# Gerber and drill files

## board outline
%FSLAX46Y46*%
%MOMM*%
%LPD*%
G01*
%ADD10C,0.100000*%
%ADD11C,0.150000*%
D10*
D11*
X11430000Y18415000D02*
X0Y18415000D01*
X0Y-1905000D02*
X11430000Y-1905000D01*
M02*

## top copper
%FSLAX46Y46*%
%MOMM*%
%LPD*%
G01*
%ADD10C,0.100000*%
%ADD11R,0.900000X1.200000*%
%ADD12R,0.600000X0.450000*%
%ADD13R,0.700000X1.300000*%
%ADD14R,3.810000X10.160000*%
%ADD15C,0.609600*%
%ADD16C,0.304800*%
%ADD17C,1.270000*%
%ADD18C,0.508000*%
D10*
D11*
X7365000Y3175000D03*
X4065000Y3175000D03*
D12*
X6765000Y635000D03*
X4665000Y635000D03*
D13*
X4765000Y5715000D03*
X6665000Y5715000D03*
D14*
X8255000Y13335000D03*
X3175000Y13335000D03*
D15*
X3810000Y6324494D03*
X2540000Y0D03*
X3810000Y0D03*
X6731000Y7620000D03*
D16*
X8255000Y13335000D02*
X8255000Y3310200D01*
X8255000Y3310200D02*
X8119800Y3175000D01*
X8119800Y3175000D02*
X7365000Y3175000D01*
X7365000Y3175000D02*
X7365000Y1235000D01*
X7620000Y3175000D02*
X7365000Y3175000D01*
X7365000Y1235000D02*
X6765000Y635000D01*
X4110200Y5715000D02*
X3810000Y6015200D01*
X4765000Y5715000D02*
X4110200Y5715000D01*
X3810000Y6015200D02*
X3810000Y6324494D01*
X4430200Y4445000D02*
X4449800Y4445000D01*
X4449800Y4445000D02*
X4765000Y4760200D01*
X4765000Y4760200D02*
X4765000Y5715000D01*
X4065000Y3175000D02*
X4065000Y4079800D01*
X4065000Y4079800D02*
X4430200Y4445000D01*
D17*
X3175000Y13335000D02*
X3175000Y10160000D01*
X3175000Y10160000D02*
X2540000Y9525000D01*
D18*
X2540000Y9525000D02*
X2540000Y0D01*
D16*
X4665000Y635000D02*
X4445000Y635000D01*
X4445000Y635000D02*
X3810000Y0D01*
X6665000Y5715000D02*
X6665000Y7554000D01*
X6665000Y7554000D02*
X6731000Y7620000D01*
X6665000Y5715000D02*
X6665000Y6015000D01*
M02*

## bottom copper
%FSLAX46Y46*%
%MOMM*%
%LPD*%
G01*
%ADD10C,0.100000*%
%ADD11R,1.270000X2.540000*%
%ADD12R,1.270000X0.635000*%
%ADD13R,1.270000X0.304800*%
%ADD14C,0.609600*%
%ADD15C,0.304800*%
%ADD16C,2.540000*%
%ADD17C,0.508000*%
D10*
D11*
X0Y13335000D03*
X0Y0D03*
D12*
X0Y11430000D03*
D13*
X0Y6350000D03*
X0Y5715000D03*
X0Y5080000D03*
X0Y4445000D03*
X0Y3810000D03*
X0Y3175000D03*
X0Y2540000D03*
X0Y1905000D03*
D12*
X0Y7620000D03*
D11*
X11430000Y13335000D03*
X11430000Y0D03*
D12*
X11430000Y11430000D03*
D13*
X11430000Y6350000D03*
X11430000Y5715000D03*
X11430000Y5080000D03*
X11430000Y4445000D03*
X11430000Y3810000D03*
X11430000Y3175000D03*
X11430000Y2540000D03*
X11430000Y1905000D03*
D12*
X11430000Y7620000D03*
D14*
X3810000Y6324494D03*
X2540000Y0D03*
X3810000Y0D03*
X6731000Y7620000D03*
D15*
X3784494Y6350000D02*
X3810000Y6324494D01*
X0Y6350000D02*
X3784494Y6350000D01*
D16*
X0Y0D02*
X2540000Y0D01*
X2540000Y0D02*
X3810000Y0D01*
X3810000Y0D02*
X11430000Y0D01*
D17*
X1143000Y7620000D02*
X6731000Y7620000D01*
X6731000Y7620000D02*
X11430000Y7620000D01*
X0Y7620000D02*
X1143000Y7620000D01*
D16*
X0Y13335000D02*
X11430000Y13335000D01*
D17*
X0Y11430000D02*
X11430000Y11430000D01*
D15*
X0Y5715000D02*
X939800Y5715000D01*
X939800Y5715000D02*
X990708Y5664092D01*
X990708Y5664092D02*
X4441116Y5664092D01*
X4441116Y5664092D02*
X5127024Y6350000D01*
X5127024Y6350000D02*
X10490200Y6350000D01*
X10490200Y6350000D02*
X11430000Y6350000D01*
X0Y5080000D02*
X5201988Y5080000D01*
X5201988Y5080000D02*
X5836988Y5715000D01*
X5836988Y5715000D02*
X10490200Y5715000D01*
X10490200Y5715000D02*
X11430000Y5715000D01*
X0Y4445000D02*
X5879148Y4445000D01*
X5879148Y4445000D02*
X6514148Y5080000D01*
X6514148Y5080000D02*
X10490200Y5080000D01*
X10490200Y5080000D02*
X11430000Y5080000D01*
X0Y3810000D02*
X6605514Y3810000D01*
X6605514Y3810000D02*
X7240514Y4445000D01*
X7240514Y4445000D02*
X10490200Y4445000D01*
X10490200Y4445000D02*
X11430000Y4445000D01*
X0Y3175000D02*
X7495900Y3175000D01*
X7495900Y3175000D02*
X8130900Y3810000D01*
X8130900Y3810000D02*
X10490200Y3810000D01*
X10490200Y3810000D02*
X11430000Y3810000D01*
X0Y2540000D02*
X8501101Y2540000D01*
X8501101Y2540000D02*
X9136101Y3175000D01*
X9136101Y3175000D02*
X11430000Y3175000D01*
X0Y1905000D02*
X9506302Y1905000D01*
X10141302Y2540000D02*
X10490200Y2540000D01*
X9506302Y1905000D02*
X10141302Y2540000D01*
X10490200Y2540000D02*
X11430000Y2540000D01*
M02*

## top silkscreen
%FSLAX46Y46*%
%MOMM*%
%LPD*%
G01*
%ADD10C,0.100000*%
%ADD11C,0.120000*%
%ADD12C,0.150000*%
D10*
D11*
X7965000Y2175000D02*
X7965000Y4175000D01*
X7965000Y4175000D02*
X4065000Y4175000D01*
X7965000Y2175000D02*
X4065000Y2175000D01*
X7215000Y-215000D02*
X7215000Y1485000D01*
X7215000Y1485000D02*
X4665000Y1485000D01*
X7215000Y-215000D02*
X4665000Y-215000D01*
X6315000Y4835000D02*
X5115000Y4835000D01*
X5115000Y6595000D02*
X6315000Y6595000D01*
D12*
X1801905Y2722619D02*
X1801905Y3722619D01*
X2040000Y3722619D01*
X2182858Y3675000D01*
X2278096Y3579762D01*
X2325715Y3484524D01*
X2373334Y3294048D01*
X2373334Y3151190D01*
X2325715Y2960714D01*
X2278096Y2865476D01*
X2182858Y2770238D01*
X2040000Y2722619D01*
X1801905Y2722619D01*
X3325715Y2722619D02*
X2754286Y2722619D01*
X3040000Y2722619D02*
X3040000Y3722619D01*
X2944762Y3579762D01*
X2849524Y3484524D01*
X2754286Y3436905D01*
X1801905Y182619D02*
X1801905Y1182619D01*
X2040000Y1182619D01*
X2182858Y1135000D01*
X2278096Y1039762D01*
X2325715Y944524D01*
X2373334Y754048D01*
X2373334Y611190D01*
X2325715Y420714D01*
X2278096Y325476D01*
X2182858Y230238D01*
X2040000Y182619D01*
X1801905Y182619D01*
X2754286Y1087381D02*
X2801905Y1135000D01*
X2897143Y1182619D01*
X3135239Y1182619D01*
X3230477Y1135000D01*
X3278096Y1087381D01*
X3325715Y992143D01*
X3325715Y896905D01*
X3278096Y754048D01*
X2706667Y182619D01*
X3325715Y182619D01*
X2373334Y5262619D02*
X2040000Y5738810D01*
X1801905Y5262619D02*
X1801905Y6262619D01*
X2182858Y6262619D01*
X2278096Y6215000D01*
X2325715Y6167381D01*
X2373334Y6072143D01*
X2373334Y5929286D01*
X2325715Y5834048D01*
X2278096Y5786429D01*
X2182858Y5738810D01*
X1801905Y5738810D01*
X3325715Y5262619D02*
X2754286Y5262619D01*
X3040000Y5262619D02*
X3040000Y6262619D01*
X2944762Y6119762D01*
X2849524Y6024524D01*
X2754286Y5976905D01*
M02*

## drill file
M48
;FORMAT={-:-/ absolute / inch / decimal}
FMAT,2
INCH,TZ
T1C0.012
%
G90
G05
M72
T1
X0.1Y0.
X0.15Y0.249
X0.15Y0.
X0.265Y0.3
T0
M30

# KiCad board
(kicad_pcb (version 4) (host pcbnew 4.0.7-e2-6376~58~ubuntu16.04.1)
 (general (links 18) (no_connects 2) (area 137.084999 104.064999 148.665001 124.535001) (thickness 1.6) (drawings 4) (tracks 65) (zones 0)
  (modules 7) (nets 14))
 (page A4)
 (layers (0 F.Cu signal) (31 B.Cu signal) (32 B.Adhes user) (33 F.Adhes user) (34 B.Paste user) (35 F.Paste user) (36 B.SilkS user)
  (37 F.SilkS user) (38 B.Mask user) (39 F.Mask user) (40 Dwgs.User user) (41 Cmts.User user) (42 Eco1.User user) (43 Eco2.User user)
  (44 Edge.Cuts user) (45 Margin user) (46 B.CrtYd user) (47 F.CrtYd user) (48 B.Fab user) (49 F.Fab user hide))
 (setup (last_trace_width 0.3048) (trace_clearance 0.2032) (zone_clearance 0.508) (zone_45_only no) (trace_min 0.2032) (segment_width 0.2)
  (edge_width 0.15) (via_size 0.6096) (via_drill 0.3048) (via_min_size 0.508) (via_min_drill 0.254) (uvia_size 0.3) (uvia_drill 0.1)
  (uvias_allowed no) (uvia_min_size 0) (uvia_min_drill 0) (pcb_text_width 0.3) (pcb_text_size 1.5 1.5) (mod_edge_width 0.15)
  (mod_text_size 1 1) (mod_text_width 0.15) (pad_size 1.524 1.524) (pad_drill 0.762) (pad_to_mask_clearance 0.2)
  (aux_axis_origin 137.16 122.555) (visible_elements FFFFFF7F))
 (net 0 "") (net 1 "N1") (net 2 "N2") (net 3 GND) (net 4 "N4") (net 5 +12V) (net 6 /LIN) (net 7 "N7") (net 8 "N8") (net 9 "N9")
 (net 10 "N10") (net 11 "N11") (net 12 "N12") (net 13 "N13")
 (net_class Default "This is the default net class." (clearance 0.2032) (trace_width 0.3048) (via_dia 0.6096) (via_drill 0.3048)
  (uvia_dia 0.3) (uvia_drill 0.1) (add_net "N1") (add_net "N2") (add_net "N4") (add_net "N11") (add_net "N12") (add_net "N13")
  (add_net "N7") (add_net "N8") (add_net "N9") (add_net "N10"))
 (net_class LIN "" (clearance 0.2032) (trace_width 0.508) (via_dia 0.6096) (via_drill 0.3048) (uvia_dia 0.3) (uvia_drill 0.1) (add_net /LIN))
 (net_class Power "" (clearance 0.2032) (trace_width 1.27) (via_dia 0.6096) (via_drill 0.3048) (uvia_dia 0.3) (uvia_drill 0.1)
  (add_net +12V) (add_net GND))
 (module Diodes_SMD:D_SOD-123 (layer F.Cu) (at 142.875 119.38 180)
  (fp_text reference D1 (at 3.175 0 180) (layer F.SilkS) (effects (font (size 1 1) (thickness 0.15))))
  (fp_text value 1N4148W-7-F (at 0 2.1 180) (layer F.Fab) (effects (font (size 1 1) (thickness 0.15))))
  (fp_line (start -2.25 -1) (end -2.25 1) (layer F.SilkS) (width 0.12))
  (fp_line (start -2.25 1) (end 1.65 1) (layer F.SilkS) (width 0.12))
  (fp_line (start -2.25 -1) (end 1.65 -1) (layer F.SilkS) (width 0.12))
  (pad 1 smd rect (at -1.65 0 180) (size 0.9 1.2) (layers F.Cu F.Paste F.Mask) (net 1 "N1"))
  (pad 2 smd rect (at 1.65 0 180) (size 0.9 1.2) (layers F.Cu F.Paste F.Mask) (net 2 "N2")))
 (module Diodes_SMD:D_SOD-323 (layer F.Cu) (at 142.875 121.92 180)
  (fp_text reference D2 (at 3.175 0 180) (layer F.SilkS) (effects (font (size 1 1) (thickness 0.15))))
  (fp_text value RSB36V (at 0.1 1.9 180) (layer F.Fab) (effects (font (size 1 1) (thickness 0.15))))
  (fp_line (start -1.5 -0.85) (end -1.5 0.85) (layer F.SilkS) (width 0.12))
  (fp_line (start -1.5 0.85) (end 1.05 0.85) (layer F.SilkS) (width 0.12))
  (fp_line (start -1.5 -0.85) (end 1.05 -0.85) (layer F.SilkS) (width 0.12))
  (pad 1 smd rect (at -1.05 0 180) (size 0.6 0.45) (layers F.Cu F.Paste F.Mask) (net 1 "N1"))
  (pad 2 smd rect (at 1.05 0 180) (size 0.6 0.45) (layers F.Cu F.Paste F.Mask) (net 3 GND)))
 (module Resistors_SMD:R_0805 (layer F.Cu) (at 142.875 116.84)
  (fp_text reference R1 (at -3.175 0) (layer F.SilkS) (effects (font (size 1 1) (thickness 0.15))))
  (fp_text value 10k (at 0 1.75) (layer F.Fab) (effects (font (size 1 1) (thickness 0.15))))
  (fp_line (start 0.6 0.88) (end -0.6 0.88) (layer F.SilkS) (width 0.12))
  (fp_line (start -0.6 -0.88) (end 0.6 -0.88) (layer F.SilkS) (width 0.12))
  (pad 1 smd rect (at -0.95 0) (size 0.7 1.3) (layers F.Cu F.Paste F.Mask) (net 2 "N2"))
  (pad 2 smd rect (at 0.95 0) (size 0.7 1.3) (layers F.Cu F.Paste F.Mask) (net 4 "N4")))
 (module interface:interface (layer F.Cu) (at 137.16 104.775)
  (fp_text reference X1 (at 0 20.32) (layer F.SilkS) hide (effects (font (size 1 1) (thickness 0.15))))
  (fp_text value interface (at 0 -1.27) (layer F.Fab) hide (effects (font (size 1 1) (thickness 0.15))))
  (pad 1 smd rect (at 0 4.445) (size 1.27 2.54) (layers B.Cu) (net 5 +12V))
  (pad 2 smd rect (at 0 17.78) (size 1.27 2.54) (layers B.Cu) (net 3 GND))
  (pad 3 smd rect (at 0 6.35) (size 1.27 0.635) (layers B.Cu) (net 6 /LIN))
  (pad 5 smd rect (at 0 11.43) (size 1.27 0.3048) (layers B.Cu) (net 2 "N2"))
  (pad 6 smd rect (at 0 12.065) (size 1.27 0.3048) (layers B.Cu) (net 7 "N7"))
  (pad 7 smd rect (at 0 12.7) (size 1.27 0.3048) (layers B.Cu) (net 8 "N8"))
  (pad 8 smd rect (at 0 13.335) (size 1.27 0.3048) (layers B.Cu) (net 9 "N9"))
  (pad 9 smd rect (at 0 13.97) (size 1.27 0.3048) (layers B.Cu) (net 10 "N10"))
  (pad 10 smd rect (at 0 14.605) (size 1.27 0.3048) (layers B.Cu) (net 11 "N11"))
  (pad 11 smd rect (at 0 15.24) (size 1.27 0.3048) (layers B.Cu) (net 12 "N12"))
  (pad 12 smd rect (at 0 15.875) (size 1.27 0.3048) (layers B.Cu) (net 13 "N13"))
  (pad 4 smd rect (at 0 10.16) (size 1.27 0.635) (layers B.Cu) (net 4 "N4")))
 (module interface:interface (layer F.Cu) (at 148.59 104.775)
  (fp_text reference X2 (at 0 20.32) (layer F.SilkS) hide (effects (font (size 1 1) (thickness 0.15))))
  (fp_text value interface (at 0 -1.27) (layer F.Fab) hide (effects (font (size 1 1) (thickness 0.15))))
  (pad 1 smd rect (at 0 4.445) (size 1.27 2.54) (layers B.Cu) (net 5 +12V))
  (pad 2 smd rect (at 0 17.78) (size 1.27 2.54) (layers B.Cu) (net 3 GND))
  (pad 3 smd rect (at 0 6.35) (size 1.27 0.635) (layers B.Cu) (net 6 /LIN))
  (pad 5 smd rect (at 0 11.43) (size 1.27 0.3048) (layers B.Cu) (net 7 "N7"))
  (pad 6 smd rect (at 0 12.065) (size 1.27 0.3048) (layers B.Cu) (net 8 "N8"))
  (pad 7 smd rect (at 0 12.7) (size 1.27 0.3048) (layers B.Cu) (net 9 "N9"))
  (pad 8 smd rect (at 0 13.335) (size 1.27 0.3048) (layers B.Cu) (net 10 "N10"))
  (pad 9 smd rect (at 0 13.97) (size 1.27 0.3048) (layers B.Cu) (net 11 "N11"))
  (pad 10 smd rect (at 0 14.605) (size 1.27 0.3048) (layers B.Cu) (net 12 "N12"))
  (pad 11 smd rect (at 0 15.24) (size 1.27 0.3048) (layers B.Cu) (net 13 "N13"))
  (pad 12 smd rect (at 0 15.875) (size 1.27 0.3048) (layers B.Cu))
  (pad 4 smd rect (at 0 10.16) (size 1.27 0.635) (layers B.Cu) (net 4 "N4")))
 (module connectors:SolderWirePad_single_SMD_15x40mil (layer F.Cu) (at 145.415 109.22)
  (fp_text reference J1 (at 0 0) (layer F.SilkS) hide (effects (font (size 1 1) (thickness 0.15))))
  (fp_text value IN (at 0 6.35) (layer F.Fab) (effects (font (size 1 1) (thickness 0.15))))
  (pad 1 smd rect (at 0 0) (size 3.81 10.16) (layers F.Cu F.Paste F.Mask) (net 1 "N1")))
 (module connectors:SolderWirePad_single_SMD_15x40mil (layer F.Cu) (at 140.335 109.22)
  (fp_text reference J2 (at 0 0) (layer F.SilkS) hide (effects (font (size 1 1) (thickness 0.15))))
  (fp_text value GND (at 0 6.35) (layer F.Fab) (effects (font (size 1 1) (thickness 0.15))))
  (pad 1 smd rect (at 0 0) (size 3.81 10.16) (layers F.Cu F.Paste F.Mask) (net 3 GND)))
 (gr_line (start 148.59 104.14) (end 137.16 104.14) (layer Edge.Cuts) (width 0.15))
 (gr_line (start 137.16 124.46) (end 148.59 124.46) (layer Edge.Cuts) (width 0.15))
 (segment (start 145.415 109.22) (end 145.415 119.2448) (width 0.3048) (layer F.Cu) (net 1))
 (segment (start 145.415 119.2448) (end 145.2798 119.38) (width 0.3048) (layer F.Cu) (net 1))
 (segment (start 145.2798 119.38) (end 144.525 119.38) (width 0.3048) (layer F.Cu) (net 1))
 (segment (start 144.525 119.38) (end 144.525 121.32) (width 0.3048) (layer F.Cu) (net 1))
 (segment (start 144.78 119.38) (end 144.525 119.38) (width 0.3048) (layer F.Cu) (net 1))
 (segment (start 144.525 121.32) (end 143.925 121.92) (width 0.3048) (layer F.Cu) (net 1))
 (segment (start 140.944494 116.205) (end 140.97 116.230506) (width 0.3048) (layer B.Cu) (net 2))
 (segment (start 137.16 116.205) (end 140.944494 116.205) (width 0.3048) (layer B.Cu) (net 2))
 (segment (start 141.2702 116.84) (end 140.97 116.5398) (width 0.3048) (layer F.Cu) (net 2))
 (segment (start 141.925 116.84) (end 141.2702 116.84) (width 0.3048) (layer F.Cu) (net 2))
 (segment (start 140.97 116.5398) (end 140.97 116.230506) (width 0.3048) (layer F.Cu) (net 2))
 (via (at 140.97 116.230506) (size 0.6096) (drill 0.3048) (layers F.Cu B.Cu) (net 2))
 (segment (start 141.5902 118.11) (end 141.6098 118.11) (width 0.3048) (layer F.Cu) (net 2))
 (segment (start 141.6098 118.11) (end 141.925 117.7948) (width 0.3048) (layer F.Cu) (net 2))
 (segment (start 141.925 117.7948) (end 141.925 116.84) (width 0.3048) (layer F.Cu) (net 2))
 (segment (start 141.225 119.38) (end 141.225 118.4752) (width 0.3048) (layer F.Cu) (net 2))
 (segment (start 141.225 118.4752) (end 141.5902 118.11) (width 0.3048) (layer F.Cu) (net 2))
 (segment (start 137.16 122.555) (end 139.7 122.555) (width 2.54) (layer B.Cu) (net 3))
 (segment (start 139.7 122.555) (end 140.97 122.555) (width 2.54) (layer B.Cu) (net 3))
 (segment (start 140.335 109.22) (end 140.335 112.395) (width 1.27) (layer F.Cu) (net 3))
 (segment (start 140.335 112.395) (end 139.7 113.03) (width 1.27) (layer F.Cu) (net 3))
 (segment (start 139.7 113.03) (end 139.7 122.555) (width 0.508) (layer F.Cu) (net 3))
 (via (at 139.7 122.555) (size 0.6096) (drill 0.3048) (layers F.Cu B.Cu) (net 3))
 (segment (start 140.97 122.555) (end 148.59 122.555) (width 2.54) (layer B.Cu) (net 3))
 (segment (start 141.825 121.92) (end 141.605 121.92) (width 0.3048) (layer F.Cu) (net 3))
 (segment (start 141.605 121.92) (end 140.97 122.555) (width 0.3048) (layer F.Cu) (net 3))
 (via (at 140.97 122.555) (size 0.6096) (drill 0.3048) (layers F.Cu B.Cu) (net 3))
 (segment (start 143.825 116.84) (end 143.825 115.001) (width 0.3048) (layer F.Cu) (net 4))
 (via (at 143.891 114.935) (size 0.6096) (drill 0.3048) (layers F.Cu B.Cu) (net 4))
 (segment (start 143.825 115.001) (end 143.891 114.935) (width 0.3048) (layer F.Cu) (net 4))
 (segment (start 138.303 114.935) (end 143.891 114.935) (width 0.508) (layer B.Cu) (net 4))
 (segment (start 143.891 114.935) (end 148.59 114.935) (width 0.508) (layer B.Cu) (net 4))
 (segment (start 137.16 114.935) (end 138.303 114.935) (width 0.508) (layer B.Cu) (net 4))
 (segment (start 143.825 116.84) (end 143.825 116.54) (width 0.3048) (layer F.Cu) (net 4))
 (segment (start 137.16 109.22) (end 148.59 109.22) (width 2.54) (layer B.Cu) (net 5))
 (segment (start 137.16 111.125) (end 148.59 111.125) (width 0.508) (layer B.Cu) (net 6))
 (segment (start 137.16 116.84) (end 138.0998 116.84) (width 0.3048) (layer B.Cu) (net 7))
 (segment (start 138.0998 116.84) (end 138.150708 116.890908) (width 0.3048) (layer B.Cu) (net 7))
 (segment (start 138.150708 116.890908) (end 141.601116 116.890908) (width 0.3048) (layer B.Cu) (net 7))
 (segment (start 141.601116 116.890908) (end 142.287024 116.205) (width 0.3048) (layer B.Cu) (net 7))
 (segment (start 142.287024 116.205) (end 147.6502 116.205) (width 0.3048) (layer B.Cu) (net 7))
 (segment (start 147.6502 116.205) (end 148.59 116.205) (width 0.3048) (layer B.Cu) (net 7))
 (segment (start 137.16 117.475) (end 142.361988 117.475) (width 0.3048) (layer B.Cu) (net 8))
 (segment (start 142.361988 117.475) (end 142.996988 116.84) (width 0.3048) (layer B.Cu) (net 8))
 (segment (start 142.996988 116.84) (end 147.6502 116.84) (width 0.3048) (layer B.Cu) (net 8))
 (segment (start 147.6502 116.84) (end 148.59 116.84) (width 0.3048) (layer B.Cu) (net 8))
 (segment (start 137.16 118.11) (end 143.039148 118.11) (width 0.3048) (layer B.Cu) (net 9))
 (segment (start 143.039148 118.11) (end 143.674148 117.475) (width 0.3048) (layer B.Cu) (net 9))
 (segment (start 143.674148 117.475) (end 147.6502 117.475) (width 0.3048) (layer B.Cu) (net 9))
 (segment (start 147.6502 117.475) (end 148.59 117.475) (width 0.3048) (layer B.Cu) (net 9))
 (segment (start 137.16 118.745) (end 143.765514 118.745) (width 0.3048) (layer B.Cu) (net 10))
 (segment (start 143.765514 118.745) (end 144.400514 118.11) (width 0.3048) (layer B.Cu) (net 10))
 (segment (start 144.400514 118.11) (end 147.6502 118.11) (width 0.3048) (layer B.Cu) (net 10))
 (segment (start 147.6502 118.11) (end 148.59 118.11) (width 0.3048) (layer B.Cu) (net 10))
 (segment (start 137.16 119.38) (end 144.6559 119.38) (width 0.3048) (layer B.Cu) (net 11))
 (segment (start 144.6559 119.38) (end 145.2909 118.745) (width 0.3048) (layer B.Cu) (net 11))
 (segment (start 145.2909 118.745) (end 147.6502 118.745) (width 0.3048) (layer B.Cu) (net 11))
 (segment (start 147.6502 118.745) (end 148.59 118.745) (width 0.3048) (layer B.Cu) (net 11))
 (segment (start 137.16 120.015) (end 145.661101 120.015) (width 0.3048) (layer B.Cu) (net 12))
 (segment (start 145.661101 120.015) (end 146.296101 119.38) (width 0.3048) (layer B.Cu) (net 12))
 (segment (start 146.296101 119.38) (end 148.59 119.38) (width 0.3048) (layer B.Cu) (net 12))
 (segment (start 137.16 120.65) (end 146.666302 120.65) (width 0.3048) (layer B.Cu) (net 13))
 (segment (start 147.301302 120.015) (end 147.6502 120.015) (width 0.3048) (layer B.Cu) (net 13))
 (segment (start 146.666302 120.65) (end 147.301302 120.015) (width 0.3048) (layer B.Cu) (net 13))
 (segment (start 147.6502 120.015) (end 148.59 120.015) (width 0.3048) (layer B.Cu) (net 13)))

